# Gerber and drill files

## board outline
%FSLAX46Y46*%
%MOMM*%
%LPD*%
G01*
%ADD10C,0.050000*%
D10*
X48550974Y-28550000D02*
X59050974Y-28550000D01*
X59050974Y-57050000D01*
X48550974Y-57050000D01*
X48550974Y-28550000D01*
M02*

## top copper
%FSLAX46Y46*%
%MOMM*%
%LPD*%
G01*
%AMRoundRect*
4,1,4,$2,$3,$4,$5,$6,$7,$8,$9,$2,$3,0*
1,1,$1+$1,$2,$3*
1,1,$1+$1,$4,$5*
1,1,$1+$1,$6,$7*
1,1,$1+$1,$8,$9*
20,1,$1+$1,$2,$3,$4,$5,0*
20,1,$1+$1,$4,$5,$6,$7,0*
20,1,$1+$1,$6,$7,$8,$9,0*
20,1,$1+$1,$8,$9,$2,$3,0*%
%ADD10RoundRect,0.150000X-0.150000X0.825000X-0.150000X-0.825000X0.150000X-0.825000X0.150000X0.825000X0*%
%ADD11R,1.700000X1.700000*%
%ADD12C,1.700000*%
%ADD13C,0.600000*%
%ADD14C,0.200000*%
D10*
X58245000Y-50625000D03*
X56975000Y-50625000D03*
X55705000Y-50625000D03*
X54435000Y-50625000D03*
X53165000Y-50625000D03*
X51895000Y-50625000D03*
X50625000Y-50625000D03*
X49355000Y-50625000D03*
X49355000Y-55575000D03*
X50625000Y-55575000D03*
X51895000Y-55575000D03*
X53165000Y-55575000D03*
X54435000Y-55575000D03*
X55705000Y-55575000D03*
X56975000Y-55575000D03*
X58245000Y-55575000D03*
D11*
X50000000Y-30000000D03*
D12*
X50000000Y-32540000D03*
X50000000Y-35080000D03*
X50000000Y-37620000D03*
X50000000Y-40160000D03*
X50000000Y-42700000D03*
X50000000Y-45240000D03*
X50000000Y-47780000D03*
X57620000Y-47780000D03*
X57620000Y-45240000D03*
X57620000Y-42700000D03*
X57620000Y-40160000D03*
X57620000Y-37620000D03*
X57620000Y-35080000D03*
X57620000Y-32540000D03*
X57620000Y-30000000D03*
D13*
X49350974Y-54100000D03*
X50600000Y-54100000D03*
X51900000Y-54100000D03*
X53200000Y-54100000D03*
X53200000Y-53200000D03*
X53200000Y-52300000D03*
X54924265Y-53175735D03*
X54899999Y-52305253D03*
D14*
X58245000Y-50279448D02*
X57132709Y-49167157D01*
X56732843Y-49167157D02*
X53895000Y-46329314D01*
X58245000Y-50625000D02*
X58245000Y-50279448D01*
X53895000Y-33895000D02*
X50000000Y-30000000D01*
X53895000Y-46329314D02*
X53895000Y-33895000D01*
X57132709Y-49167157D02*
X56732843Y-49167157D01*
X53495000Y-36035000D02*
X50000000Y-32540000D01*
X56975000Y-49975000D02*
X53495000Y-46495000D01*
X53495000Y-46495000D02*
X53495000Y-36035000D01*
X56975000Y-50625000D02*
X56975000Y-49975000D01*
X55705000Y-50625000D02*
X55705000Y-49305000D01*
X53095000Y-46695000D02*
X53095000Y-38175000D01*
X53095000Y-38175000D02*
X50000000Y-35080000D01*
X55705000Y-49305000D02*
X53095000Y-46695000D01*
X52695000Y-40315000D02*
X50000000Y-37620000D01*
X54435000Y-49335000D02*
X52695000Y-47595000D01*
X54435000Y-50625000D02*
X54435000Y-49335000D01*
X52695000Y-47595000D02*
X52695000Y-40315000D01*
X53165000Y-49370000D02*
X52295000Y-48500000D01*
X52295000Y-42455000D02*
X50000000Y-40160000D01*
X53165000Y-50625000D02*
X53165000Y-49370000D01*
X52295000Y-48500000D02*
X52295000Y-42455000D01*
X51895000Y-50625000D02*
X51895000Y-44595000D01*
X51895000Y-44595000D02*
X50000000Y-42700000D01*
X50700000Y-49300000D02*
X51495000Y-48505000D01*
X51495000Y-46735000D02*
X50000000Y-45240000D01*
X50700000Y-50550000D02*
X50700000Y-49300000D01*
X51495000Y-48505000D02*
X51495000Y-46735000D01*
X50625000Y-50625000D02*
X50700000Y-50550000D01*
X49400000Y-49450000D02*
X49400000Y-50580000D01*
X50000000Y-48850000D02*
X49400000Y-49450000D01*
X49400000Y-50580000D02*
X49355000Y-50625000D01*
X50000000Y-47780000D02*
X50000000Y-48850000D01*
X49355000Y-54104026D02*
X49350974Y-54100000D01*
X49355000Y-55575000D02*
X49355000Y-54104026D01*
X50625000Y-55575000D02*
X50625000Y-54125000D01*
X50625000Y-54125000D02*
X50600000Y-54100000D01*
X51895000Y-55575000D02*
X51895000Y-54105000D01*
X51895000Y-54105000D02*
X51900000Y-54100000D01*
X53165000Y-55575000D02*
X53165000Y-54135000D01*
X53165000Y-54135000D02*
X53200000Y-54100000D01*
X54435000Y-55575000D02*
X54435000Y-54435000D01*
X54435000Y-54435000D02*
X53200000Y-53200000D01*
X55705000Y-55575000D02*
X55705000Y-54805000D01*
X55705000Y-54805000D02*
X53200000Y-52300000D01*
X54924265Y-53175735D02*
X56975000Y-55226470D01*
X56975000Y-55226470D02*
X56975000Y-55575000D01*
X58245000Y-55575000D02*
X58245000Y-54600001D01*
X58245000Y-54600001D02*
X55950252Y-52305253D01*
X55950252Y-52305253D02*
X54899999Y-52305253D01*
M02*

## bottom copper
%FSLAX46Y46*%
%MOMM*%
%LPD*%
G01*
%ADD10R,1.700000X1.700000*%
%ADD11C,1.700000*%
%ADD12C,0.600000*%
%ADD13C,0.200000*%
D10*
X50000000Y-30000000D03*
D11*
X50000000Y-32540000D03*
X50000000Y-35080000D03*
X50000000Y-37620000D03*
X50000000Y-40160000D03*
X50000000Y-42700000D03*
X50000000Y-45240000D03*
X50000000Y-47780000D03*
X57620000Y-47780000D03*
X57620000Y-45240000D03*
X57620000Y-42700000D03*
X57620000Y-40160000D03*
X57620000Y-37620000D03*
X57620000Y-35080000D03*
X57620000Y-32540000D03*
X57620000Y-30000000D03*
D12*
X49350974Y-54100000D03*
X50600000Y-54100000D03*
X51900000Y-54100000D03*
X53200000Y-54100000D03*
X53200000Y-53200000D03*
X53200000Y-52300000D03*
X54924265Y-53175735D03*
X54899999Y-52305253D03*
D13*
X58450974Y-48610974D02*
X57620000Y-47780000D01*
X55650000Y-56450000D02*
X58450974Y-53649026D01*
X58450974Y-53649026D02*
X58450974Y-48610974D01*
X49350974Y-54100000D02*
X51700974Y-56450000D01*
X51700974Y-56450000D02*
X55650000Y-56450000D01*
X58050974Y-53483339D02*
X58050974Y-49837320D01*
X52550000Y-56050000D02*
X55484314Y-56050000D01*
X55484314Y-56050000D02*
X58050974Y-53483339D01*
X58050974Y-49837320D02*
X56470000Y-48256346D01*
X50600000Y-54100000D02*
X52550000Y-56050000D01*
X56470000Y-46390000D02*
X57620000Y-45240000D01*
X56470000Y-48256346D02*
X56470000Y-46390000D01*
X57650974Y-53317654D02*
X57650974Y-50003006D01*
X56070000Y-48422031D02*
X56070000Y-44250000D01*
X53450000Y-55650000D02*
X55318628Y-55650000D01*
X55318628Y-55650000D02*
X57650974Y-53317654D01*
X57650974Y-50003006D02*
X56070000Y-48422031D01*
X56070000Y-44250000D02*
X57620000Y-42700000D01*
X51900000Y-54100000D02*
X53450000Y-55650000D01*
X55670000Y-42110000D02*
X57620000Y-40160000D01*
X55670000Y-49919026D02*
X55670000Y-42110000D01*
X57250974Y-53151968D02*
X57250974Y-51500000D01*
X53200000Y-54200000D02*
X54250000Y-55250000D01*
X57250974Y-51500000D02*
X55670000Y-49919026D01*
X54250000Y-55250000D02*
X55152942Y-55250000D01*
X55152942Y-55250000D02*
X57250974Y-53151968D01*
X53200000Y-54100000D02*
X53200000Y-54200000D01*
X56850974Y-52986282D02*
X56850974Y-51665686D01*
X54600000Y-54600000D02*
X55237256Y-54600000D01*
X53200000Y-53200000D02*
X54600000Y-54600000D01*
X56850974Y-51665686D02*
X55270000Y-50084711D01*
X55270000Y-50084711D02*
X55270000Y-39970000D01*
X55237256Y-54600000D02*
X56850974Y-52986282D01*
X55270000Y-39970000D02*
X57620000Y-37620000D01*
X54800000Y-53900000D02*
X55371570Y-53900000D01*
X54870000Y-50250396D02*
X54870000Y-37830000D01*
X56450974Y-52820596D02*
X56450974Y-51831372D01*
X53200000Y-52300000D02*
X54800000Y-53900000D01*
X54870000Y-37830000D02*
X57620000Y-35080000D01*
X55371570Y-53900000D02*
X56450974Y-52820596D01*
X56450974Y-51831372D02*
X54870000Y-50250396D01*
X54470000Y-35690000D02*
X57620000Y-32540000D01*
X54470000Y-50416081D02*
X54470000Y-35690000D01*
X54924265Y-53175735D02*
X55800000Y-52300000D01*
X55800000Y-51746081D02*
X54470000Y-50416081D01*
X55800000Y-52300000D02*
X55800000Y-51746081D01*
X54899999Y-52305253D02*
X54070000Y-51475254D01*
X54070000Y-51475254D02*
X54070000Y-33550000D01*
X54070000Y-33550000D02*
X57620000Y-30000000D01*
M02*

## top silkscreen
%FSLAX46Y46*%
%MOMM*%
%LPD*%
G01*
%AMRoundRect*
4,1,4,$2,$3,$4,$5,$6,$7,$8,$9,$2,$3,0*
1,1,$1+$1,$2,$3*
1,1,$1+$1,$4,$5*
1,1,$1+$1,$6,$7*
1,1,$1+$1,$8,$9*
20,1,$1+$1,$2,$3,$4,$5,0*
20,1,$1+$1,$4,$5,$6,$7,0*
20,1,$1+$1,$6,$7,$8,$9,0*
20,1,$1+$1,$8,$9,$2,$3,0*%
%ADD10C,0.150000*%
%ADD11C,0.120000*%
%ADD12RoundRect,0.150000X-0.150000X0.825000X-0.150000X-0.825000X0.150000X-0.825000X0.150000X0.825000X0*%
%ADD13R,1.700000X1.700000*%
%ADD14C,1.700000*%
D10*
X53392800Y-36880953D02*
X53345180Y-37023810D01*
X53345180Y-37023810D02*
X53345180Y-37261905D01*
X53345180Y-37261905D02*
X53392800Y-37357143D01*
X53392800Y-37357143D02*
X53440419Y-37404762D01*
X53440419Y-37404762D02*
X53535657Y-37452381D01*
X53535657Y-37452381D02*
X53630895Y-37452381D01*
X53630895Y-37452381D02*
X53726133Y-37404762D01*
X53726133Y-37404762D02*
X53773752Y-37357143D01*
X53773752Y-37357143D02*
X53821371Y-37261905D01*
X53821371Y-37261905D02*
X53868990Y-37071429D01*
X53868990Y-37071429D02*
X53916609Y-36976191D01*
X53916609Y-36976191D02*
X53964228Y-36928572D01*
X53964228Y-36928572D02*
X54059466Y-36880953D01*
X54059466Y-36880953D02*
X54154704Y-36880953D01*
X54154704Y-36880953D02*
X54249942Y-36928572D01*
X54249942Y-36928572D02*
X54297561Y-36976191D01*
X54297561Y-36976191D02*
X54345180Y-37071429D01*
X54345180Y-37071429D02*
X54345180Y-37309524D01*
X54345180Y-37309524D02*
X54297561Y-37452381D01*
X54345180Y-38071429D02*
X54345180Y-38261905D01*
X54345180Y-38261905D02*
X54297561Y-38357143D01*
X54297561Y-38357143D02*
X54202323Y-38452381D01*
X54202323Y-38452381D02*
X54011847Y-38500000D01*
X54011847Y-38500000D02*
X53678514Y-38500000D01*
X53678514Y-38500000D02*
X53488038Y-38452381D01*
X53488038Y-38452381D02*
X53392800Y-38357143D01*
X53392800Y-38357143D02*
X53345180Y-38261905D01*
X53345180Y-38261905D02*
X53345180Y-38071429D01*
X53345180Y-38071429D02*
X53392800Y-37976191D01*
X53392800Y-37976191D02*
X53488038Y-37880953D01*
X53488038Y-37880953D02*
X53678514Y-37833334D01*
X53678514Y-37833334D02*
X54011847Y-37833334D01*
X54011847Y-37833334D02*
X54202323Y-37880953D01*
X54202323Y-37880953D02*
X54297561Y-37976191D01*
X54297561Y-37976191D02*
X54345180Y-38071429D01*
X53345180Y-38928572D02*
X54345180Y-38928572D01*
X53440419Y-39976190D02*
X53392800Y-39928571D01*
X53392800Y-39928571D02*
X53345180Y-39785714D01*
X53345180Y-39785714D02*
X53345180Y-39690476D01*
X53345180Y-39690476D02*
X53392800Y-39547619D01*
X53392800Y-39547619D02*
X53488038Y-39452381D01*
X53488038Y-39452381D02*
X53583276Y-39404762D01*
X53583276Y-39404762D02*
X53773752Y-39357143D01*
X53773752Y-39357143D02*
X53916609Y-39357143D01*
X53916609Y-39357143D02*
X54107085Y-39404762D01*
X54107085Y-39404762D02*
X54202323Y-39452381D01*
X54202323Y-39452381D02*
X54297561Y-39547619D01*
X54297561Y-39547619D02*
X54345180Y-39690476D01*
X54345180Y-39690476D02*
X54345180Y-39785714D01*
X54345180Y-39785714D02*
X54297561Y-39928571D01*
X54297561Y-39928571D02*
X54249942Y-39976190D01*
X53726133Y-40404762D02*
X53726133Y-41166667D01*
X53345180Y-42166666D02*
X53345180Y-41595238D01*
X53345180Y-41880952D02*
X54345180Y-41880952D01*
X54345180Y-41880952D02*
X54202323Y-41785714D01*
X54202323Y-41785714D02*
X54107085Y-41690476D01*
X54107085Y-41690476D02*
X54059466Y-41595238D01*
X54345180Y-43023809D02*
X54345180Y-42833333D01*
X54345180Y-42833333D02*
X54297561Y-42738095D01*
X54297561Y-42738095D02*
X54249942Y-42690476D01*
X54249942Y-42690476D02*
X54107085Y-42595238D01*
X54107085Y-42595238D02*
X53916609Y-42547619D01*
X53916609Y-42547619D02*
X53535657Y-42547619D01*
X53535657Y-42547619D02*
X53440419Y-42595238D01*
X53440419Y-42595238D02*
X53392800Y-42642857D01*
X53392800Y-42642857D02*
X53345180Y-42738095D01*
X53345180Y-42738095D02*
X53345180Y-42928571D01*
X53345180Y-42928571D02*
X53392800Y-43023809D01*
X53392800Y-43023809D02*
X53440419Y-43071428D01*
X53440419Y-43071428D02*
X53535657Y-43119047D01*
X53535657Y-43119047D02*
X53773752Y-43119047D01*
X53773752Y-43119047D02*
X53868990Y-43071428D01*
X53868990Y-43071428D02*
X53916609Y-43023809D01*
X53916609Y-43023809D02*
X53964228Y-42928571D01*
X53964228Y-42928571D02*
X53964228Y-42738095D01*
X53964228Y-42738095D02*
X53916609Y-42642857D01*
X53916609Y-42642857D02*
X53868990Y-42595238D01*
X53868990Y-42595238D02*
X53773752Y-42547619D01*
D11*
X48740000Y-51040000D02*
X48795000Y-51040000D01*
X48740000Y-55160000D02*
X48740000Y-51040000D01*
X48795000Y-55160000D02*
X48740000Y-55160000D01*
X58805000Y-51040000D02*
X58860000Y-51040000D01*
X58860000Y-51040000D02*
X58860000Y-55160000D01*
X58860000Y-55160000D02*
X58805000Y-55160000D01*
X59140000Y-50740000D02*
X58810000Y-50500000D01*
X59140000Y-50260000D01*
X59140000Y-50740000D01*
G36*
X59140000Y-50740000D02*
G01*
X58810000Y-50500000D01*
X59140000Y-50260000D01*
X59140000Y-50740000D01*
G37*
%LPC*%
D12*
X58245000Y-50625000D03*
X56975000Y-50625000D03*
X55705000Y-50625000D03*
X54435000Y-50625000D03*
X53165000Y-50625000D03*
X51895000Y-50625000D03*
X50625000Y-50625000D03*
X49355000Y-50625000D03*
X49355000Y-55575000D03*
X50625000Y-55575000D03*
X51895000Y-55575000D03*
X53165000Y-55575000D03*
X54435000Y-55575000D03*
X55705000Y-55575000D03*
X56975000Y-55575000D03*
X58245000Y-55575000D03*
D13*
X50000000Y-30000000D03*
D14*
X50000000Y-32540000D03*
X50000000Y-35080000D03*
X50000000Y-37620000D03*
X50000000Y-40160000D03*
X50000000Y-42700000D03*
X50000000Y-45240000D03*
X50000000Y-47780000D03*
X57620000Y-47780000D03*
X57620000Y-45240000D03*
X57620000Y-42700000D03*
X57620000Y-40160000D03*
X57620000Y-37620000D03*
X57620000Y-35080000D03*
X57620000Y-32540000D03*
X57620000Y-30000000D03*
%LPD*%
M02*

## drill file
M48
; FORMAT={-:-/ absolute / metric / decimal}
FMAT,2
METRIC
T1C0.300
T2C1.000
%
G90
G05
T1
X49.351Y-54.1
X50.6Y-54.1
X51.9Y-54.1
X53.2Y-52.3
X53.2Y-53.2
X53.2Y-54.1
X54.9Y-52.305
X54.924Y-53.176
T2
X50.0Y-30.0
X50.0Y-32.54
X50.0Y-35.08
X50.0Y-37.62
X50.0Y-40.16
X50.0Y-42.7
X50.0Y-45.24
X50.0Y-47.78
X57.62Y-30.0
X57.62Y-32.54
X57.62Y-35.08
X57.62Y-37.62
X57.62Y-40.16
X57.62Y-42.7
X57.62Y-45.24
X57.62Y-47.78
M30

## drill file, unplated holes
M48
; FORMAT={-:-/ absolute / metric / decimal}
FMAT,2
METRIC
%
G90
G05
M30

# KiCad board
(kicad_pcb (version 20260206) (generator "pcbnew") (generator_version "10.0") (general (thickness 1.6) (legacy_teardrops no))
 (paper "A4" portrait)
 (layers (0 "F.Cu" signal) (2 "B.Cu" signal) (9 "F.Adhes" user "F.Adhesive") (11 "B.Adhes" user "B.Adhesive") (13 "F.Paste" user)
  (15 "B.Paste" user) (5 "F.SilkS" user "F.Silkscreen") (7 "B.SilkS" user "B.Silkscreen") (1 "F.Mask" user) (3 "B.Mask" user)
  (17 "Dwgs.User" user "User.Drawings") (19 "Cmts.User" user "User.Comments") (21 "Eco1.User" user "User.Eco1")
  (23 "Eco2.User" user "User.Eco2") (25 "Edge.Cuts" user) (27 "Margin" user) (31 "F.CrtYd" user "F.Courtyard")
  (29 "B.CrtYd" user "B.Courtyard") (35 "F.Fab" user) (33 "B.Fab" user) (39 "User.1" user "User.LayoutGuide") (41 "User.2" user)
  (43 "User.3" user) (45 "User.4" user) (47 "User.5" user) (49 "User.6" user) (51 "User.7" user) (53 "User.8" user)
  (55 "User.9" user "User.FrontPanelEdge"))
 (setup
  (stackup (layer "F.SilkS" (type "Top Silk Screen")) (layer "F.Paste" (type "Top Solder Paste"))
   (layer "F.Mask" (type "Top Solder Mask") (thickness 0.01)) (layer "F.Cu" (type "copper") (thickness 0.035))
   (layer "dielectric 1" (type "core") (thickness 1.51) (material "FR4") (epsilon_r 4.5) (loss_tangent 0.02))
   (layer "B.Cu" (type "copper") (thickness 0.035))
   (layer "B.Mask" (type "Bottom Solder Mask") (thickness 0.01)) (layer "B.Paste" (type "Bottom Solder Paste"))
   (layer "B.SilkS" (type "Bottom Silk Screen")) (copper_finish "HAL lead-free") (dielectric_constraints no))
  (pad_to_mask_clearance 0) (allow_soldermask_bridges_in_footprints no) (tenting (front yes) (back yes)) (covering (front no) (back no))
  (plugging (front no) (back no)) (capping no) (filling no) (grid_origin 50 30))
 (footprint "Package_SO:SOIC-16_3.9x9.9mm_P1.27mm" (layer "F.Cu") (at 53.8 53.1 -90)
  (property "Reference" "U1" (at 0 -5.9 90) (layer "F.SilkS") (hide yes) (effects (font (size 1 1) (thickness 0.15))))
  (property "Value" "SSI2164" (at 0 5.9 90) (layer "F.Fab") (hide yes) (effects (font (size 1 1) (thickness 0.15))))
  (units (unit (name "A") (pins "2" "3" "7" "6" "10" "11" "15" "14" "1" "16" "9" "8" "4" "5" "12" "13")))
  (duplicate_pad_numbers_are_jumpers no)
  (fp_line (start -2.06 5.06) (end -2.06 5.005) (stroke (width 0.12) (type solid)) (layer "F.SilkS"))
  (fp_line (start 2.06 5.06) (end -2.06 5.06) (stroke (width 0.12) (type solid)) (layer "F.SilkS"))
  (fp_line (start 2.06 5.005) (end 2.06 5.06) (stroke (width 0.12) (type solid)) (layer "F.SilkS"))
  (fp_line (start -2.06 -5.005) (end -2.06 -5.06) (stroke (width 0.12) (type solid)) (layer "F.SilkS"))
  (fp_line (start -2.06 -5.06) (end 2.06 -5.06) (stroke (width 0.12) (type solid)) (layer "F.SilkS"))
  (fp_line (start 2.06 -5.06) (end 2.06 -5.005) (stroke (width 0.12) (type solid)) (layer "F.SilkS"))
  (fp_poly (pts (xy -2.6 -5.01) (xy -2.84 -5.34) (xy -2.36 -5.34)) (stroke (width 0.12) (type solid)) (fill yes) (layer "F.SilkS"))
  (pad "1" smd roundrect (at -2.475 -4.445 270) (size 1.95 0.6) (layers "F.Cu" "F.Mask" "F.Paste") (roundrect_rratio 0.25)
   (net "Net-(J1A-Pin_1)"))
  (pad "2" smd roundrect (at -2.475 -3.175 270) (size 1.95 0.6) (layers "F.Cu" "F.Mask" "F.Paste") (roundrect_rratio 0.25)
   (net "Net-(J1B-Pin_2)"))
  (pad "3" smd roundrect (at -2.475 -1.905 270) (size 1.95 0.6) (layers "F.Cu" "F.Mask" "F.Paste") (roundrect_rratio 0.25)
   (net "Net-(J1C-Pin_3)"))
  (pad "4" smd roundrect (at -2.475 -0.635 270) (size 1.95 0.6) (layers "F.Cu" "F.Mask" "F.Paste") (roundrect_rratio 0.25)
   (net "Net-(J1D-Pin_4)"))
  (pad "5" smd roundrect (at -2.475 0.635 270) (size 1.95 0.6) (layers "F.Cu" "F.Mask" "F.Paste") (roundrect_rratio 0.25)
   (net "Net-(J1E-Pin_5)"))
  (pad "6" smd roundrect (at -2.475 1.905 270) (size 1.95 0.6) (layers "F.Cu" "F.Mask" "F.Paste") (roundrect_rratio 0.25)
   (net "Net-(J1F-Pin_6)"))
  (pad "7" smd roundrect (at -2.475 3.175 270) (size 1.95 0.6) (layers "F.Cu" "F.Mask" "F.Paste") (roundrect_rratio 0.25)
   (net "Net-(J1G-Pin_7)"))
  (pad "8" smd roundrect (at -2.475 4.445 270) (size 1.95 0.6) (layers "F.Cu" "F.Mask" "F.Paste") (roundrect_rratio 0.25)
   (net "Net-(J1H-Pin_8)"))
  (pad "9" smd roundrect (at 2.475 4.445 270) (size 1.95 0.6) (layers "F.Cu" "F.Mask" "F.Paste") (roundrect_rratio 0.25)
   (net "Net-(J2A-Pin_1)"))
  (pad "10" smd roundrect (at 2.475 3.175 270) (size 1.95 0.6) (layers "F.Cu" "F.Mask" "F.Paste") (roundrect_rratio 0.25)
   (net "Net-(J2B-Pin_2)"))
  (pad "11" smd roundrect (at 2.475 1.905 270) (size 1.95 0.6) (layers "F.Cu" "F.Mask" "F.Paste") (roundrect_rratio 0.25)
   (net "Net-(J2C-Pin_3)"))
  (pad "12" smd roundrect (at 2.475 0.635 270) (size 1.95 0.6) (layers "F.Cu" "F.Mask" "F.Paste") (roundrect_rratio 0.25)
   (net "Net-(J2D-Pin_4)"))
  (pad "13" smd roundrect (at 2.475 -0.635 270) (size 1.95 0.6) (layers "F.Cu" "F.Mask" "F.Paste") (roundrect_rratio 0.25)
   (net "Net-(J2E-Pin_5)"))
  (pad "14" smd roundrect (at 2.475 -1.905 270) (size 1.95 0.6) (layers "F.Cu" "F.Mask" "F.Paste") (roundrect_rratio 0.25)
   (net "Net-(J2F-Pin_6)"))
  (pad "15" smd roundrect (at 2.475 -3.175 270) (size 1.95 0.6) (layers "F.Cu" "F.Mask" "F.Paste") (roundrect_rratio 0.25)
   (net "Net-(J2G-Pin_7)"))
  (pad "16" smd roundrect (at 2.475 -4.445 270) (size 1.95 0.6) (layers "F.Cu" "F.Mask" "F.Paste") (roundrect_rratio 0.25)
   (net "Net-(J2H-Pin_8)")))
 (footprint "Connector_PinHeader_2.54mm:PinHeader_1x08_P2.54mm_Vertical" (layer "B.Cu") (at 50 30 180)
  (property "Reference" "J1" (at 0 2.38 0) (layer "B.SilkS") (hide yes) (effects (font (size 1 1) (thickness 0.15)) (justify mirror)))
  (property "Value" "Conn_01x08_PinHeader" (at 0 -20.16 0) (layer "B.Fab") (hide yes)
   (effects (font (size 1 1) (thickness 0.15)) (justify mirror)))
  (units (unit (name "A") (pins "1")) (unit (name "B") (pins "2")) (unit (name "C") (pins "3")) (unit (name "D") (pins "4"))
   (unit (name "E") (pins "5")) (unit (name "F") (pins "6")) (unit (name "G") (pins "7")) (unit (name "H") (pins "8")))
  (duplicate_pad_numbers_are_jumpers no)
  (pad "1" thru_hole rect (at 0 0 180) (size 1.7 1.7) (drill 1) (layers "*.Cu" "*.Mask") (remove_unused_layers no) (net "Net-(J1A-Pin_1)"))
  (pad "2" thru_hole circle (at 0 -2.54 180) (size 1.7 1.7) (drill 1) (layers "*.Cu" "*.Mask") (remove_unused_layers no)
   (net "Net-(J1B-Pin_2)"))
  (pad "3" thru_hole circle (at 0 -5.08 180) (size 1.7 1.7) (drill 1) (layers "*.Cu" "*.Mask") (remove_unused_layers no)
   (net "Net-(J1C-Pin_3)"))
  (pad "4" thru_hole circle (at 0 -7.62 180) (size 1.7 1.7) (drill 1) (layers "*.Cu" "*.Mask") (remove_unused_layers no)
   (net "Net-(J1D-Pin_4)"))
  (pad "5" thru_hole circle (at 0 -10.16 180) (size 1.7 1.7) (drill 1) (layers "*.Cu" "*.Mask") (remove_unused_layers no)
   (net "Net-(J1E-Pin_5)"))
  (pad "6" thru_hole circle (at 0 -12.7 180) (size 1.7 1.7) (drill 1) (layers "*.Cu" "*.Mask") (remove_unused_layers no)
   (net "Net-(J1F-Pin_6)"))
  (pad "7" thru_hole circle (at 0 -15.24 180) (size 1.7 1.7) (drill 1) (layers "*.Cu" "*.Mask") (remove_unused_layers no)
   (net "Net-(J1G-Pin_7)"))
  (pad "8" thru_hole circle (at 0 -17.78 180) (size 1.7 1.7) (drill 1) (layers "*.Cu" "*.Mask") (remove_unused_layers no)
   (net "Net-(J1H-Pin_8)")))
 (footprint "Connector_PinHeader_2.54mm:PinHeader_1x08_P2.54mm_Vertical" (layer "B.Cu") (at 57.62 47.78)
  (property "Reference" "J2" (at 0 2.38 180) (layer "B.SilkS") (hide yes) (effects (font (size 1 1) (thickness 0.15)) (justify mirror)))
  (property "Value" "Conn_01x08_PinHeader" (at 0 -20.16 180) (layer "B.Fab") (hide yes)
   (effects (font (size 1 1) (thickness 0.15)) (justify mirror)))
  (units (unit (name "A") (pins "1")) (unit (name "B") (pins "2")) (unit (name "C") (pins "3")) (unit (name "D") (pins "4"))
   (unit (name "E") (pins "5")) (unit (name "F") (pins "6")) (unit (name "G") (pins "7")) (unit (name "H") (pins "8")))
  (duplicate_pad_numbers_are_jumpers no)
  (pad "1" thru_hole circle (at 0 0) (size 1.7 1.7) (drill 1) (layers "*.Cu" "*.Mask") (remove_unused_layers no) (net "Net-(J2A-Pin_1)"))
  (pad "2" thru_hole circle (at 0 -2.54) (size 1.7 1.7) (drill 1) (layers "*.Cu" "*.Mask") (remove_unused_layers no) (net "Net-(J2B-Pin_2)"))
  (pad "3" thru_hole circle (at 0 -5.08) (size 1.7 1.7) (drill 1) (layers "*.Cu" "*.Mask") (remove_unused_layers no) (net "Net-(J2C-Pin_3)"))
  (pad "4" thru_hole circle (at 0 -7.62) (size 1.7 1.7) (drill 1) (layers "*.Cu" "*.Mask") (remove_unused_layers no) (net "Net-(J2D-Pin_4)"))
  (pad "5" thru_hole circle (at 0 -10.16) (size 1.7 1.7) (drill 1) (layers "*.Cu" "*.Mask") (remove_unused_layers no)
   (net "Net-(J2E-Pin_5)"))
  (pad "6" thru_hole circle (at 0 -12.7) (size 1.7 1.7) (drill 1) (layers "*.Cu" "*.Mask") (remove_unused_layers no) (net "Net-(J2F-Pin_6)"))
  (pad "7" thru_hole circle (at 0 -15.24) (size 1.7 1.7) (drill 1) (layers "*.Cu" "*.Mask") (remove_unused_layers no)
   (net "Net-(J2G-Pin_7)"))
  (pad "8" thru_hole circle (at 0 -17.78) (size 1.7 1.7) (drill 1) (layers "*.Cu" "*.Mask") (remove_unused_layers no)
   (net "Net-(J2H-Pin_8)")))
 (gr_rect (start 48.550974 28.55) (end 59.050974 57.05) (stroke (width 0.05) (type solid)) (fill no) (layer "Edge.Cuts"))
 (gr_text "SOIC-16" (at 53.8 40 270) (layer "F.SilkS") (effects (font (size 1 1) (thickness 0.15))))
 (segment (start 58.245 50.279448) (end 57.132709 49.167157) (width 0.2) (layer "F.Cu") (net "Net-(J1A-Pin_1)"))
 (segment (start 56.732843 49.167157) (end 53.895 46.329314) (width 0.2) (layer "F.Cu") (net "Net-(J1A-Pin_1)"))
 (segment (start 58.245 50.625) (end 58.245 50.279448) (width 0.2) (layer "F.Cu") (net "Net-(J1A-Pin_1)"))
 (segment (start 53.895 33.895) (end 50 30) (width 0.2) (layer "F.Cu") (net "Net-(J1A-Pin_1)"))
 (segment (start 53.895 46.329314) (end 53.895 33.895) (width 0.2) (layer "F.Cu") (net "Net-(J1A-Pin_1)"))
 (segment (start 57.132709 49.167157) (end 56.732843 49.167157) (width 0.2) (layer "F.Cu") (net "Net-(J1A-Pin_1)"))
 (segment (start 53.495 36.035) (end 50 32.54) (width 0.2) (layer "F.Cu") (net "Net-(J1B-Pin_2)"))
 (segment (start 56.975 49.975) (end 53.495 46.495) (width 0.2) (layer "F.Cu") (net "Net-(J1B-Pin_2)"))
 (segment (start 53.495 46.495) (end 53.495 36.035) (width 0.2) (layer "F.Cu") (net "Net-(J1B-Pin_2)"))
 (segment (start 56.975 50.625) (end 56.975 49.975) (width 0.2) (layer "F.Cu") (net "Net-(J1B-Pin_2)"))
 (segment (start 55.705 50.625) (end 55.705 49.305) (width 0.2) (layer "F.Cu") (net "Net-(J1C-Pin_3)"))
 (segment (start 53.095 46.695) (end 53.095 38.175) (width 0.2) (layer "F.Cu") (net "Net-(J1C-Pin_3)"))
 (segment (start 53.095 38.175) (end 50 35.08) (width 0.2) (layer "F.Cu") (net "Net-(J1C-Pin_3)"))
 (segment (start 55.705 49.305) (end 53.095 46.695) (width 0.2) (layer "F.Cu") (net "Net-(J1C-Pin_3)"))
 (segment (start 52.695 40.315) (end 50 37.62) (width 0.2) (layer "F.Cu") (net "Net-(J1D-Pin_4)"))
 (segment (start 54.435 49.335) (end 52.695 47.595) (width 0.2) (layer "F.Cu") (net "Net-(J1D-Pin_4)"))
 (segment (start 54.435 50.625) (end 54.435 49.335) (width 0.2) (layer "F.Cu") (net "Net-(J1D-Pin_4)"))
 (segment (start 52.695 47.595) (end 52.695 40.315) (width 0.2) (layer "F.Cu") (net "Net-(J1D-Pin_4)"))
 (segment (start 53.165 49.37) (end 52.295 48.5) (width 0.2) (layer "F.Cu") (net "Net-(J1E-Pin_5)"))
 (segment (start 52.295 42.455) (end 50 40.16) (width 0.2) (layer "F.Cu") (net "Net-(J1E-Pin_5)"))
 (segment (start 53.165 50.625) (end 53.165 49.37) (width 0.2) (layer "F.Cu") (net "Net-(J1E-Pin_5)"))
 (segment (start 52.295 48.5) (end 52.295 42.455) (width 0.2) (layer "F.Cu") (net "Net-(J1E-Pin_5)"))
 (segment (start 51.895 50.625) (end 51.895 44.595) (width 0.2) (layer "F.Cu") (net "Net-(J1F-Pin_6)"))
 (segment (start 51.895 44.595) (end 50 42.7) (width 0.2) (layer "F.Cu") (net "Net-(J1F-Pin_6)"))
 (segment (start 50.7 49.3) (end 51.495 48.505) (width 0.2) (layer "F.Cu") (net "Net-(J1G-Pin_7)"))
 (segment (start 51.495 46.735) (end 50 45.24) (width 0.2) (layer "F.Cu") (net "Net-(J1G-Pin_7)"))
 (segment (start 50.7 50.55) (end 50.7 49.3) (width 0.2) (layer "F.Cu") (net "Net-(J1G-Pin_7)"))
 (segment (start 51.495 48.505) (end 51.495 46.735) (width 0.2) (layer "F.Cu") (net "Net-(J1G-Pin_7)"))
 (segment (start 50.625 50.625) (end 50.7 50.55) (width 0.2) (layer "F.Cu") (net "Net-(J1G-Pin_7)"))
 (segment (start 49.4 49.45) (end 49.4 50.58) (width 0.2) (layer "F.Cu") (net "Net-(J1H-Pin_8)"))
 (segment (start 50 48.85) (end 49.4 49.45) (width 0.2) (layer "F.Cu") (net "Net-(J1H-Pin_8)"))
 (segment (start 49.4 50.58) (end 49.355 50.625) (width 0.2) (layer "F.Cu") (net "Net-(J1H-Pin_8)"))
 (segment (start 50 47.78) (end 50 48.85) (width 0.2) (layer "F.Cu") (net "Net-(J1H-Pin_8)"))
 (segment (start 49.355 54.104026) (end 49.350974 54.1) (width 0.2) (layer "F.Cu") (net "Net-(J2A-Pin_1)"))
 (segment (start 49.355 55.575) (end 49.355 54.104026) (width 0.2) (layer "F.Cu") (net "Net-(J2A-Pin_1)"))
 (via (at 49.350974 54.1) (size 0.6) (drill 0.3) (layers "F.Cu" "B.Cu") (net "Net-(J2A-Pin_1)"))
 (segment (start 58.450974 48.610974) (end 57.62 47.78) (width 0.2) (layer "B.Cu") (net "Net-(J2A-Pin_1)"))
 (segment (start 55.65 56.45) (end 58.450974 53.649026) (width 0.2) (layer "B.Cu") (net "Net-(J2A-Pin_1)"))
 (segment (start 58.450974 53.649026) (end 58.450974 48.610974) (width 0.2) (layer "B.Cu") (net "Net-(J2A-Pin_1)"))
 (segment (start 49.350974 54.1) (end 51.700974 56.45) (width 0.2) (layer "B.Cu") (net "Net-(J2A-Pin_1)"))
 (segment (start 51.700974 56.45) (end 55.65 56.45) (width 0.2) (layer "B.Cu") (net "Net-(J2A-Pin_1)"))
 (segment (start 50.625 55.575) (end 50.625 54.125) (width 0.2) (layer "F.Cu") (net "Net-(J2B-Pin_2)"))
 (segment (start 50.625 54.125) (end 50.6 54.1) (width 0.2) (layer "F.Cu") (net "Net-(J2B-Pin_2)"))
 (via (at 50.6 54.1) (size 0.6) (drill 0.3) (layers "F.Cu" "B.Cu") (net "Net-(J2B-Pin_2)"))
 (segment (start 58.050974 53.483339) (end 58.050974 49.83732) (width 0.2) (layer "B.Cu") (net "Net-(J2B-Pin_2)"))
 (segment (start 52.55 56.05) (end 55.484314 56.05) (width 0.2) (layer "B.Cu") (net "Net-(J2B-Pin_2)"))
 (segment (start 55.484314 56.05) (end 58.050974 53.483339) (width 0.2) (layer "B.Cu") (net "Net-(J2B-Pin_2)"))
 (segment (start 58.050974 49.83732) (end 56.47 48.256346) (width 0.2) (layer "B.Cu") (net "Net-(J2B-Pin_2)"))
 (segment (start 50.6 54.1) (end 52.55 56.05) (width 0.2) (layer "B.Cu") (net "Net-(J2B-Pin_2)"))
 (segment (start 56.47 46.39) (end 57.62 45.24) (width 0.2) (layer "B.Cu") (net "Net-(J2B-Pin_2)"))
 (segment (start 56.47 48.256346) (end 56.47 46.39) (width 0.2) (layer "B.Cu") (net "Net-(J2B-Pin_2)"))
 (segment (start 51.895 55.575) (end 51.895 54.105) (width 0.2) (layer "F.Cu") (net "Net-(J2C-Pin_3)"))
 (segment (start 51.895 54.105) (end 51.9 54.1) (width 0.2) (layer "F.Cu") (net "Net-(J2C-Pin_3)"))
 (via (at 51.9 54.1) (size 0.6) (drill 0.3) (layers "F.Cu" "B.Cu") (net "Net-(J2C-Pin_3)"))
 (segment (start 57.650974 53.317654) (end 57.650974 50.003006) (width 0.2) (layer "B.Cu") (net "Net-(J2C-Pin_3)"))
 (segment (start 56.07 48.422031) (end 56.07 44.25) (width 0.2) (layer "B.Cu") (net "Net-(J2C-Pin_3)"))
 (segment (start 53.45 55.65) (end 55.318628 55.65) (width 0.2) (layer "B.Cu") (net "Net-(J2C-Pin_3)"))
 (segment (start 55.318628 55.65) (end 57.650974 53.317654) (width 0.2) (layer "B.Cu") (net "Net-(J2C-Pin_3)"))
 (segment (start 57.650974 50.003006) (end 56.07 48.422031) (width 0.2) (layer "B.Cu") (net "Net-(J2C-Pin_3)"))
 (segment (start 56.07 44.25) (end 57.62 42.7) (width 0.2) (layer "B.Cu") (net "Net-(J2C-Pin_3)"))
 (segment (start 51.9 54.1) (end 53.45 55.65) (width 0.2) (layer "B.Cu") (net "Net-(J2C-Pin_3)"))
 (segment (start 53.165 55.575) (end 53.165 54.135) (width 0.2) (layer "F.Cu") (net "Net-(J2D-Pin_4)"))
 (segment (start 53.165 54.135) (end 53.2 54.1) (width 0.2) (layer "F.Cu") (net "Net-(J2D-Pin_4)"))
 (via (at 53.2 54.1) (size 0.6) (drill 0.3) (layers "F.Cu" "B.Cu") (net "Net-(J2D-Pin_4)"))
 (segment (start 55.67 42.11) (end 57.62 40.16) (width 0.2) (layer "B.Cu") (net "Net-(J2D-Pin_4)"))
 (segment (start 55.67 49.919026) (end 55.67 42.11) (width 0.2) (layer "B.Cu") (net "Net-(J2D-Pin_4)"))
 (segment (start 57.250974 53.151968) (end 57.250974 51.5) (width 0.2) (layer "B.Cu") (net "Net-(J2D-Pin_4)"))
 (segment (start 53.2 54.2) (end 54.25 55.25) (width 0.2) (layer "B.Cu") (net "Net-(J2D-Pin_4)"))
 (segment (start 57.250974 51.5) (end 55.67 49.919026) (width 0.2) (layer "B.Cu") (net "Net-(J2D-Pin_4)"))
 (segment (start 54.25 55.25) (end 55.152942 55.25) (width 0.2) (layer "B.Cu") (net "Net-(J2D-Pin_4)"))
 (segment (start 55.152942 55.25) (end 57.250974 53.151968) (width 0.2) (layer "B.Cu") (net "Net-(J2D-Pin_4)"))
 (segment (start 53.2 54.1) (end 53.2 54.2) (width 0.2) (layer "B.Cu") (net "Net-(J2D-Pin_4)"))
 (segment (start 54.435 55.575) (end 54.435 54.435) (width 0.2) (layer "F.Cu") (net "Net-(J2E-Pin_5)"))
 (segment (start 54.435 54.435) (end 53.2 53.2) (width 0.2) (layer "F.Cu") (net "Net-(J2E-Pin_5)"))
 (via (at 53.2 53.2) (size 0.6) (drill 0.3) (layers "F.Cu" "B.Cu") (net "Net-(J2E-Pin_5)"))
 (segment (start 56.850974 52.986282) (end 56.850974 51.665686) (width 0.2) (layer "B.Cu") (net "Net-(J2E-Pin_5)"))
 (segment (start 54.6 54.6) (end 55.237256 54.6) (width 0.2) (layer "B.Cu") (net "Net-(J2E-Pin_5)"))
 (segment (start 53.2 53.2) (end 54.6 54.6) (width 0.2) (layer "B.Cu") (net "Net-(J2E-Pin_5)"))
 (segment (start 56.850974 51.665686) (end 55.27 50.084711) (width 0.2) (layer "B.Cu") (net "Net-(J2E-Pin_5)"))
 (segment (start 55.27 50.084711) (end 55.27 39.97) (width 0.2) (layer "B.Cu") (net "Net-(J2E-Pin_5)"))
 (segment (start 55.237256 54.6) (end 56.850974 52.986282) (width 0.2) (layer "B.Cu") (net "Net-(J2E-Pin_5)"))
 (segment (start 55.27 39.97) (end 57.62 37.62) (width 0.2) (layer "B.Cu") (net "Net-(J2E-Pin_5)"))
 (segment (start 55.705 55.575) (end 55.705 54.805) (width 0.2) (layer "F.Cu") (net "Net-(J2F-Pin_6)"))
 (segment (start 55.705 54.805) (end 53.2 52.3) (width 0.2) (layer "F.Cu") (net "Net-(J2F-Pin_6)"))
 (via (at 53.2 52.3) (size 0.6) (drill 0.3) (layers "F.Cu" "B.Cu") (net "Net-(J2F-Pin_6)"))
 (segment (start 54.8 53.9) (end 55.37157 53.9) (width 0.2) (layer "B.Cu") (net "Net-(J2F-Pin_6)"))
 (segment (start 54.87 50.250396) (end 54.87 37.83) (width 0.2) (layer "B.Cu") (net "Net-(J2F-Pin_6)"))
 (segment (start 56.450974 52.820596) (end 56.450974 51.831372) (width 0.2) (layer "B.Cu") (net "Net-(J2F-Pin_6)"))
 (segment (start 53.2 52.3) (end 54.8 53.9) (width 0.2) (layer "B.Cu") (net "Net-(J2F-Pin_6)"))
 (segment (start 54.87 37.83) (end 57.62 35.08) (width 0.2) (layer "B.Cu") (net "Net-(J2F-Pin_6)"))
 (segment (start 55.37157 53.9) (end 56.450974 52.820596) (width 0.2) (layer "B.Cu") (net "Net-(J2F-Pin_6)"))
 (segment (start 56.450974 51.831372) (end 54.87 50.250396) (width 0.2) (layer "B.Cu") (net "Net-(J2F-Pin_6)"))
 (segment (start 54.924265 53.175735) (end 56.975 55.22647) (width 0.2) (layer "F.Cu") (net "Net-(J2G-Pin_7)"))
 (segment (start 56.975 55.22647) (end 56.975 55.575) (width 0.2) (layer "F.Cu") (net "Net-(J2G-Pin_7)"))
 (via (at 54.924265 53.175735) (size 0.6) (drill 0.3) (layers "F.Cu" "B.Cu") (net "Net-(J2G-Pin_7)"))
 (segment (start 54.47 35.69) (end 57.62 32.54) (width 0.2) (layer "B.Cu") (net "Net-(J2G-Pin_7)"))
 (segment (start 54.47 50.416081) (end 54.47 35.69) (width 0.2) (layer "B.Cu") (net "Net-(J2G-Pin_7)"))
 (segment (start 54.924265 53.175735) (end 55.8 52.3) (width 0.2) (layer "B.Cu") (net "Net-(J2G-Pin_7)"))
 (segment (start 55.8 51.746081) (end 54.47 50.416081) (width 0.2) (layer "B.Cu") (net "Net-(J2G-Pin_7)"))
 (segment (start 55.8 52.3) (end 55.8 51.746081) (width 0.2) (layer "B.Cu") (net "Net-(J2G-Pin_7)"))
 (segment (start 58.245 55.575) (end 58.245 54.600001) (width 0.2) (layer "F.Cu") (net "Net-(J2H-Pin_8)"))
 (segment (start 58.245 54.600001) (end 55.950252 52.305253) (width 0.2) (layer "F.Cu") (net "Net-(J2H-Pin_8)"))
 (segment (start 55.950252 52.305253) (end 54.899999 52.305253) (width 0.2) (layer "F.Cu") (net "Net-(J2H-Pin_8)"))
 (via (at 54.899999 52.305253) (size 0.6) (drill 0.3) (layers "F.Cu" "B.Cu") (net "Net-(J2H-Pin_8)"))
 (segment (start 54.899999 52.305253) (end 54.07 51.475254) (width 0.2) (layer "B.Cu") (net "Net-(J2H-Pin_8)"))
 (segment (start 54.07 51.475254) (end 54.07 33.55) (width 0.2) (layer "B.Cu") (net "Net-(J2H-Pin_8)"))
 (segment (start 54.07 33.55) (end 57.62 30) (width 0.2) (layer "B.Cu") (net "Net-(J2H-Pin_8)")))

